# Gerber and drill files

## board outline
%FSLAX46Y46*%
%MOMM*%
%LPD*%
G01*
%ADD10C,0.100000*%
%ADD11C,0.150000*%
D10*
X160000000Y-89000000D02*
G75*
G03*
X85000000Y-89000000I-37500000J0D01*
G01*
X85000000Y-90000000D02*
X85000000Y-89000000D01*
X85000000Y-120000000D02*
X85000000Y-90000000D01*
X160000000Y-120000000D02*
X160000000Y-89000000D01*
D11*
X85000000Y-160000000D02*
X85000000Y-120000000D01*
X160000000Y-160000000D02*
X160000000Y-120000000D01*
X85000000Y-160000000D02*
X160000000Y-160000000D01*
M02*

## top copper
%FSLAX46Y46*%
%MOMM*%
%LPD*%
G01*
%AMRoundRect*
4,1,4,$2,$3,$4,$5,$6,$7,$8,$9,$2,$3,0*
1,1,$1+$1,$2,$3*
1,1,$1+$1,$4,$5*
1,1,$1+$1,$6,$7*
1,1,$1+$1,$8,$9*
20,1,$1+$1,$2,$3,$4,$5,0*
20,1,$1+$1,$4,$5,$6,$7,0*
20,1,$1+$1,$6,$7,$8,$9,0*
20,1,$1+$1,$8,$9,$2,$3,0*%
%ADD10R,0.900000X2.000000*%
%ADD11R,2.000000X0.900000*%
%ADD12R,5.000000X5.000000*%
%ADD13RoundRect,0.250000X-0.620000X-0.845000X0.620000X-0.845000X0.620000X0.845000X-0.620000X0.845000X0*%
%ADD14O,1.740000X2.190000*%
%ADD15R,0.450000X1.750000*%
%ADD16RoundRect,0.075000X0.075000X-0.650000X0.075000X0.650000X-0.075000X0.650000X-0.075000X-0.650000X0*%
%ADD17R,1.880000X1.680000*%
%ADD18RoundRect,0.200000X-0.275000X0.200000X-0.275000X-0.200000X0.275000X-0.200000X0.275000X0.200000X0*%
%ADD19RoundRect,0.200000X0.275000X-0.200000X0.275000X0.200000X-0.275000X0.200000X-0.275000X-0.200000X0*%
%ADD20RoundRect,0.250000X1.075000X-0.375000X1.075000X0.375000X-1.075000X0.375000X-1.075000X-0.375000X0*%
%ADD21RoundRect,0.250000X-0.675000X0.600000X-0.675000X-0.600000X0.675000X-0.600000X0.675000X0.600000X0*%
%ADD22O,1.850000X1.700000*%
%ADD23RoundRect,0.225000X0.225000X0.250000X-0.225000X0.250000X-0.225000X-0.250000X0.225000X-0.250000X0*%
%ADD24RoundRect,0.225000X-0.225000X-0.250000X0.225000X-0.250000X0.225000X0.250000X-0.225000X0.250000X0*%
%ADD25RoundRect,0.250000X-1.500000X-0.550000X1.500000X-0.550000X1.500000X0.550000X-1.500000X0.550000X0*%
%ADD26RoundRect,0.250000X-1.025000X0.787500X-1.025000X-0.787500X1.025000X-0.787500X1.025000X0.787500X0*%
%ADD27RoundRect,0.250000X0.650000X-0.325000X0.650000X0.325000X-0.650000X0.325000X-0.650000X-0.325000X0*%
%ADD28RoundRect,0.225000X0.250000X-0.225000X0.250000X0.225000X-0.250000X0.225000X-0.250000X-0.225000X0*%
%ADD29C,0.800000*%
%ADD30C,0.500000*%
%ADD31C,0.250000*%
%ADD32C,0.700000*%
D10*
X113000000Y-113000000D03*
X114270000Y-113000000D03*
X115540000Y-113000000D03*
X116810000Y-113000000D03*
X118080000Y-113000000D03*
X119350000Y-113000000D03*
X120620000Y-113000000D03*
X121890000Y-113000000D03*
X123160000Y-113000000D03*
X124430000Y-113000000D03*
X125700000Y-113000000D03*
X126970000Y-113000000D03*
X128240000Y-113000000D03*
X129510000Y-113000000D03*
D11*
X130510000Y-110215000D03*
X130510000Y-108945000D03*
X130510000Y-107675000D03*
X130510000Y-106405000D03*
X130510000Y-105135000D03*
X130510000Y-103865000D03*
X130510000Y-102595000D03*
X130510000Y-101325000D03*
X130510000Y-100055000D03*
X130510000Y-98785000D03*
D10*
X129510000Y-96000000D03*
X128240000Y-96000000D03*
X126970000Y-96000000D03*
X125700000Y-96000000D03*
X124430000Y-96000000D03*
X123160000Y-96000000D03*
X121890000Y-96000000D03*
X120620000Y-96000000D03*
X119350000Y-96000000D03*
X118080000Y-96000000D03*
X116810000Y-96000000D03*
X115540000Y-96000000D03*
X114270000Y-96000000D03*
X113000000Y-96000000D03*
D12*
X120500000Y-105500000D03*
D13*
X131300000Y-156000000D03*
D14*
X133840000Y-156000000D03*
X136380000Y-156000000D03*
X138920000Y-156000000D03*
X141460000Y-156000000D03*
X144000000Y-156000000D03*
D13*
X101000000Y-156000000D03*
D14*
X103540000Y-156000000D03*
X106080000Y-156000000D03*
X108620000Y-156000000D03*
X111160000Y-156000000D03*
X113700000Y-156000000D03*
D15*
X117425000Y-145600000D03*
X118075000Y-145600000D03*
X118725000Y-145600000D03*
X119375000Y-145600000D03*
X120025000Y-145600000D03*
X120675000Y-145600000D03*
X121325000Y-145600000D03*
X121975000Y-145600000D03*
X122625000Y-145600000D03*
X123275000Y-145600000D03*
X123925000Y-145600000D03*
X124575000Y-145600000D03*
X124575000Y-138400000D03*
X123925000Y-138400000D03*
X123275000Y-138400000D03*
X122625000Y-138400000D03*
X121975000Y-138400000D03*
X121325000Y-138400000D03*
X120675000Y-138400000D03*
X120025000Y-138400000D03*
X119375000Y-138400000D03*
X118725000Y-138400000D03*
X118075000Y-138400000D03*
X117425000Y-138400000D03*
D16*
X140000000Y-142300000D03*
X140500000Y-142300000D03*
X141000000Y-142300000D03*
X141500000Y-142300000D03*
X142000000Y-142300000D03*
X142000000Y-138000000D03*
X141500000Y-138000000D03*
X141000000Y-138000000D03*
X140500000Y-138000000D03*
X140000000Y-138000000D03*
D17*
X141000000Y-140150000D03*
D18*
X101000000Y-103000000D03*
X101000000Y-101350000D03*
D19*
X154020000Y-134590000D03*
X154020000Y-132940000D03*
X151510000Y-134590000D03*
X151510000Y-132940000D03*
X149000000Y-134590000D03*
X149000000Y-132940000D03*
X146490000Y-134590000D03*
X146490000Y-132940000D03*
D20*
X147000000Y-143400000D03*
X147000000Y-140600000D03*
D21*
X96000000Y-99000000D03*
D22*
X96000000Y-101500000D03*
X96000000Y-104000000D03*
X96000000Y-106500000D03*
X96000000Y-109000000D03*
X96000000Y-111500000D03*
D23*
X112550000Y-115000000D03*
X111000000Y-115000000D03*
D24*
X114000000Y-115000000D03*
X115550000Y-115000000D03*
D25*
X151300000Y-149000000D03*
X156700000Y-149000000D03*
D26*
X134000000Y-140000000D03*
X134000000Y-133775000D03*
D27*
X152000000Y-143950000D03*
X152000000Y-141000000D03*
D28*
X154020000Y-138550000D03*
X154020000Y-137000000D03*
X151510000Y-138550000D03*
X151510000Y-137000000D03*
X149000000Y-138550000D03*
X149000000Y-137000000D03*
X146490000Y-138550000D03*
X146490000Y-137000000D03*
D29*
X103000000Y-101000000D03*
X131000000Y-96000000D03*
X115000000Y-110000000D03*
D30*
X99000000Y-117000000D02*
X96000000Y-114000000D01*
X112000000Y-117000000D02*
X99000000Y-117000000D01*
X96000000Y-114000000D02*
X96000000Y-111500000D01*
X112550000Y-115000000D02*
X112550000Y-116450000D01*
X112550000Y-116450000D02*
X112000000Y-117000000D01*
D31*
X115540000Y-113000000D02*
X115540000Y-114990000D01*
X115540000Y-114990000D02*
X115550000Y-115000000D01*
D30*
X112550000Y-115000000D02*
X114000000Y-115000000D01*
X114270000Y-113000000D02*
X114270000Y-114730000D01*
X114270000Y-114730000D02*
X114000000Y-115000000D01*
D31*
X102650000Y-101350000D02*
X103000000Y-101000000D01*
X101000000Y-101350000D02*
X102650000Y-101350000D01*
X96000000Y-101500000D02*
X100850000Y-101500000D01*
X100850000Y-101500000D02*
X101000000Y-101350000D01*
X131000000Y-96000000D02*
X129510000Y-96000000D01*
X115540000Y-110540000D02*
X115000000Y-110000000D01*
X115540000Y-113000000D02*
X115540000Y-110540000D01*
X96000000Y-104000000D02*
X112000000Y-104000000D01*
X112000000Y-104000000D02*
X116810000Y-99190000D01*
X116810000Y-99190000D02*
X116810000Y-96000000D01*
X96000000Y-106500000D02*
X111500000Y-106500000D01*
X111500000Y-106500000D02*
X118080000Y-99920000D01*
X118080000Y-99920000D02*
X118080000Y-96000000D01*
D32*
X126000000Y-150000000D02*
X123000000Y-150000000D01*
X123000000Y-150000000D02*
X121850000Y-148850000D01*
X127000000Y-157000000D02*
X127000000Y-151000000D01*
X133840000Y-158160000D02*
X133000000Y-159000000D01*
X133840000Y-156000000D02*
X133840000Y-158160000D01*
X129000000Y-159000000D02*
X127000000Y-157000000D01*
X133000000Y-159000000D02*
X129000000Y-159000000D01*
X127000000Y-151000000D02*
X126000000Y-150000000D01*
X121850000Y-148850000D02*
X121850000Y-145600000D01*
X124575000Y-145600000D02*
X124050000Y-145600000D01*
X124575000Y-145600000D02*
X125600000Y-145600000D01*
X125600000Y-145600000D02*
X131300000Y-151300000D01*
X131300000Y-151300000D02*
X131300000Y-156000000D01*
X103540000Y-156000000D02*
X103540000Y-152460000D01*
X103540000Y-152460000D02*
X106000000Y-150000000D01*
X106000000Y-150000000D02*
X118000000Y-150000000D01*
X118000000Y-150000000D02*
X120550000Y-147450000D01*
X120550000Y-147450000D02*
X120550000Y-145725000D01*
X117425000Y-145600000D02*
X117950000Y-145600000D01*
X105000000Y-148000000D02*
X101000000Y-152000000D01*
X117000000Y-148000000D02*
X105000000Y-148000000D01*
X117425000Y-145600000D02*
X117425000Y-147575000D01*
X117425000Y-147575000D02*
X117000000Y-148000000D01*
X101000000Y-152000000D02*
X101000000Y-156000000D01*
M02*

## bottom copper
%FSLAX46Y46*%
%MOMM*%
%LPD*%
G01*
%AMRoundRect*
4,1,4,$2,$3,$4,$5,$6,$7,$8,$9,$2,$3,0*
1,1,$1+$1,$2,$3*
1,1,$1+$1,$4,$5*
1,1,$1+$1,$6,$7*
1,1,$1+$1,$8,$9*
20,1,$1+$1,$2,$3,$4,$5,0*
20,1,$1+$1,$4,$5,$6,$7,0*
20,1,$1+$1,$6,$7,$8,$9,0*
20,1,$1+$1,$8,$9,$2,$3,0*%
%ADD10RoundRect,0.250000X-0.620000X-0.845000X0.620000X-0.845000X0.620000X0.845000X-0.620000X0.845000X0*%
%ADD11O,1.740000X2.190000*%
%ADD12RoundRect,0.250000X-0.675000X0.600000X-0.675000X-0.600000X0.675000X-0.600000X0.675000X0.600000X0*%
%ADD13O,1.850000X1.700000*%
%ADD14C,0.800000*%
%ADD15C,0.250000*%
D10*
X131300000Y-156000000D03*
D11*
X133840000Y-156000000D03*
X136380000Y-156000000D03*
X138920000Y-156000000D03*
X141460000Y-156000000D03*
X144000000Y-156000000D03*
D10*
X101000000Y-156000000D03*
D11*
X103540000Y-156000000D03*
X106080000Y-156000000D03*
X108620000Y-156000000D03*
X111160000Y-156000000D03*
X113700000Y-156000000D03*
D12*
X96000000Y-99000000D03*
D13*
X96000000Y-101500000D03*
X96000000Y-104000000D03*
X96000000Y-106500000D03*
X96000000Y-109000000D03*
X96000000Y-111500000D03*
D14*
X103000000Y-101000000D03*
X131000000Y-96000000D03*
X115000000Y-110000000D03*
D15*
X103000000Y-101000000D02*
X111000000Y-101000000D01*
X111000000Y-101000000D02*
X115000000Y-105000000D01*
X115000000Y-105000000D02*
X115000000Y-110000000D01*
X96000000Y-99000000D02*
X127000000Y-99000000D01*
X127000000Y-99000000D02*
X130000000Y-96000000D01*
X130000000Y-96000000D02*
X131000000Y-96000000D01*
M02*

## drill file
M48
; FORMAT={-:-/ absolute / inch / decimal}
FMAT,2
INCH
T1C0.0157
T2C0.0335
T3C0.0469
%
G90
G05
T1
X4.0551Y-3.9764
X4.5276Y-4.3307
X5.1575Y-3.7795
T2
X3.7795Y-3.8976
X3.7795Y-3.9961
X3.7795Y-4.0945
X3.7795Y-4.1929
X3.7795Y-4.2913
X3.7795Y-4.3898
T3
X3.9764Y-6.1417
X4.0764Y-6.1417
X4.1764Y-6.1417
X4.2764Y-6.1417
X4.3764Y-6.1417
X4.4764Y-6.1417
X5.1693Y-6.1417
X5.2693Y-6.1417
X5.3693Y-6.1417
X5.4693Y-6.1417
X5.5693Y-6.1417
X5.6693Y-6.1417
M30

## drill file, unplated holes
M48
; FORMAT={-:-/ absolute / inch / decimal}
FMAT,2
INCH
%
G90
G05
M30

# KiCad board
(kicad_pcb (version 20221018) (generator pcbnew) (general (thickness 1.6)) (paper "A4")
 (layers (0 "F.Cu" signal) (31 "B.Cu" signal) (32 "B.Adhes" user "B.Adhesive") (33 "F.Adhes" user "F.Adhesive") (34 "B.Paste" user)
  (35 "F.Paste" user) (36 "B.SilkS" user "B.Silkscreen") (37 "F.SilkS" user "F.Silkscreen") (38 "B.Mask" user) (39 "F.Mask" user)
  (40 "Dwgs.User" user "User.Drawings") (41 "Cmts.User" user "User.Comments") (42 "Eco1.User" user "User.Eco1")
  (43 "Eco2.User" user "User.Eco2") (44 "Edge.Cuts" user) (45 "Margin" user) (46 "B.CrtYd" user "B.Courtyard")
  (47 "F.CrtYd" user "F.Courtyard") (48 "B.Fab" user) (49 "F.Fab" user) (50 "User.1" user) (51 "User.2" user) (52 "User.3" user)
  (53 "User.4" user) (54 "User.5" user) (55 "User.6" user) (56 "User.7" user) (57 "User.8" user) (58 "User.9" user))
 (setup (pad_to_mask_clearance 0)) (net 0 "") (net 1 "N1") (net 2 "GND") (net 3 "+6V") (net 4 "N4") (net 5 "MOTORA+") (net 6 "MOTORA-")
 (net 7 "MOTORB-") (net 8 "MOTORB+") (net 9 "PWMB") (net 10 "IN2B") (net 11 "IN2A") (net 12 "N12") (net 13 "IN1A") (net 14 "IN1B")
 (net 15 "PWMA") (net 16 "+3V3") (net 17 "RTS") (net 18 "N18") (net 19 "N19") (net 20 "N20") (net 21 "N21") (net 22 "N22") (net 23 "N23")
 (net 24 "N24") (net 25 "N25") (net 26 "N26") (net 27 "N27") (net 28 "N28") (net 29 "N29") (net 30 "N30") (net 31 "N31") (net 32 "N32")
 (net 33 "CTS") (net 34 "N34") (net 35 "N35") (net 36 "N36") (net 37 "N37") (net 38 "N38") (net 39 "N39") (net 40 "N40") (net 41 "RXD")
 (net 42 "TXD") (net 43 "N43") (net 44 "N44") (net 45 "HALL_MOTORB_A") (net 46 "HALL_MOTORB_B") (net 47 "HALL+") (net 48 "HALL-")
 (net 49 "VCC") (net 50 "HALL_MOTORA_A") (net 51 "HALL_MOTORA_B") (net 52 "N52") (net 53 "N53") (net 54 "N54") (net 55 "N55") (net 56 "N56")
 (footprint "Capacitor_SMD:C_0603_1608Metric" (layer "F.Cu") (at 146.49 137.775 90)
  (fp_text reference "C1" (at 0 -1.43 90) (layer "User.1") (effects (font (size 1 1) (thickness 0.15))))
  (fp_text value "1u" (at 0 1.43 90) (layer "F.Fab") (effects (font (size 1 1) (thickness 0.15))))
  (pad "1" smd roundrect (at -0.775 0 90) (size 0.9 0.95) (layers "F.Cu" "F.Paste" "F.Mask") (roundrect_rratio 0.25) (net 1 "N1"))
  (pad "2" smd roundrect (at 0.775 0 90) (size 0.9 0.95) (layers "F.Cu" "F.Paste" "F.Mask") (roundrect_rratio 0.25) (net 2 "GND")))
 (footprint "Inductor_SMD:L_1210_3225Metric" (layer "F.Cu") (at 147 142 90)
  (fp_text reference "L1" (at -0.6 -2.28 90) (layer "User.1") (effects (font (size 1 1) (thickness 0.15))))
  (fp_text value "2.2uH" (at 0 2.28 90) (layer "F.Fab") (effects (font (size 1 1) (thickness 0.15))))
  (pad "1" smd roundrect (at -1.4 0 90) (size 1.25 2.65) (layers "F.Cu" "F.Paste" "F.Mask") (roundrect_rratio 0.2) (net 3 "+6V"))
  (pad "2" smd roundrect (at 1.4 0 90) (size 1.25 2.65) (layers "F.Cu" "F.Paste" "F.Mask") (roundrect_rratio 0.2) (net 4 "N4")))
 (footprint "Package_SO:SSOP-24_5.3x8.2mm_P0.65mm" (layer "F.Cu") (at 121 142 90)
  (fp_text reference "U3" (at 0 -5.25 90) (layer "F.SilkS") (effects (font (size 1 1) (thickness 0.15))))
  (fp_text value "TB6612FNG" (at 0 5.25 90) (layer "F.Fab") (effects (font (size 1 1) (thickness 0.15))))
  (pad "1" smd rect (at -3.6 -3.575 90) (size 1.75 0.45) (layers "F.Cu" "F.Paste" "F.Mask") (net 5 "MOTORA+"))
  (pad "2" smd rect (at -3.6 -2.925 90) (size 1.75 0.45) (layers "F.Cu" "F.Paste" "F.Mask") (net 5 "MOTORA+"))
  (pad "3" smd rect (at -3.6 -2.275 90) (size 1.75 0.45) (layers "F.Cu" "F.Paste" "F.Mask") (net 2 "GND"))
  (pad "4" smd rect (at -3.6 -1.625 90) (size 1.75 0.45) (layers "F.Cu" "F.Paste" "F.Mask") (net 2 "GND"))
  (pad "5" smd rect (at -3.6 -0.975 90) (size 1.75 0.45) (layers "F.Cu" "F.Paste" "F.Mask") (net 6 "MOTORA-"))
  (pad "6" smd rect (at -3.6 -0.325 90) (size 1.75 0.45) (layers "F.Cu" "F.Paste" "F.Mask") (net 6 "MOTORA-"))
  (pad "7" smd rect (at -3.6 0.325 90) (size 1.75 0.45) (layers "F.Cu" "F.Paste" "F.Mask") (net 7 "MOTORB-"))
  (pad "8" smd rect (at -3.6 0.975 90) (size 1.75 0.45) (layers "F.Cu" "F.Paste" "F.Mask") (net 7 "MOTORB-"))
  (pad "9" smd rect (at -3.6 1.625 90) (size 1.75 0.45) (layers "F.Cu" "F.Paste" "F.Mask") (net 2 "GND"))
  (pad "10" smd rect (at -3.6 2.275 90) (size 1.75 0.45) (layers "F.Cu" "F.Paste" "F.Mask") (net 2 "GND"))
  (pad "11" smd rect (at -3.6 2.925 90) (size 1.75 0.45) (layers "F.Cu" "F.Paste" "F.Mask") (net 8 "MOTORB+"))
  (pad "12" smd rect (at -3.6 3.575 90) (size 1.75 0.45) (layers "F.Cu" "F.Paste" "F.Mask") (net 8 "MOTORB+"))
  (pad "13" smd rect (at 3.6 3.575 90) (size 1.75 0.45) (layers "F.Cu" "F.Paste" "F.Mask") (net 3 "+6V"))
  (pad "14" smd rect (at 3.6 2.925 90) (size 1.75 0.45) (layers "F.Cu" "F.Paste" "F.Mask") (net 3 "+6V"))
  (pad "15" smd rect (at 3.6 2.275 90) (size 1.75 0.45) (layers "F.Cu" "F.Paste" "F.Mask") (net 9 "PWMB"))
  (pad "16" smd rect (at 3.6 1.625 90) (size 1.75 0.45) (layers "F.Cu" "F.Paste" "F.Mask") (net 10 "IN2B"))
  (pad "17" smd rect (at 3.6 0.975 90) (size 1.75 0.45) (layers "F.Cu" "F.Paste" "F.Mask") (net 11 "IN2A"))
  (pad "18" smd rect (at 3.6 0.325 90) (size 1.75 0.45) (layers "F.Cu" "F.Paste" "F.Mask") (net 2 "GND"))
  (pad "19" smd rect (at 3.6 -0.325 90) (size 1.75 0.45) (layers "F.Cu" "F.Paste" "F.Mask") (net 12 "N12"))
  (pad "20" smd rect (at 3.6 -0.975 90) (size 1.75 0.45) (layers "F.Cu" "F.Paste" "F.Mask") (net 3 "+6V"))
  (pad "21" smd rect (at 3.6 -1.625 90) (size 1.75 0.45) (layers "F.Cu" "F.Paste" "F.Mask") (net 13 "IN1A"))
  (pad "22" smd rect (at 3.6 -2.275 90) (size 1.75 0.45) (layers "F.Cu" "F.Paste" "F.Mask") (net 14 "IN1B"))
  (pad "23" smd rect (at 3.6 -2.925 90) (size 1.75 0.45) (layers "F.Cu" "F.Paste" "F.Mask") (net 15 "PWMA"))
  (pad "24" smd rect (at 3.6 -3.575 90) (size 1.75 0.45) (layers "F.Cu" "F.Paste" "F.Mask") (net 3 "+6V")))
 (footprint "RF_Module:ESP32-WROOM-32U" (layer "F.Cu") (at 121.255 104.5 90)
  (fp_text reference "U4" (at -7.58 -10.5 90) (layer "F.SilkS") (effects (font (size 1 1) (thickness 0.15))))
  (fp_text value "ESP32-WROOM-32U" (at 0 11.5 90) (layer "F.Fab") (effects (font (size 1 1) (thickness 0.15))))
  (pad "1" smd rect (at -8.5 -8.255 90) (size 2 0.9) (layers "F.Cu" "F.Paste" "F.Mask") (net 2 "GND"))
  (pad "2" smd rect (at -8.5 -6.985 90) (size 2 0.9) (layers "F.Cu" "F.Paste" "F.Mask") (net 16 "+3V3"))
  (pad "3" smd rect (at -8.5 -5.715 90) (size 2 0.9) (layers "F.Cu" "F.Paste" "F.Mask") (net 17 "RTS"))
  (pad "4" smd rect (at -8.5 -4.445 90) (size 2 0.9) (layers "F.Cu" "F.Paste" "F.Mask") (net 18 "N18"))
  (pad "5" smd rect (at -8.5 -3.175 90) (size 2 0.9) (layers "F.Cu" "F.Paste" "F.Mask") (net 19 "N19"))
  (pad "6" smd rect (at -8.5 -1.905 90) (size 2 0.9) (layers "F.Cu" "F.Paste" "F.Mask") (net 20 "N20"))
  (pad "7" smd rect (at -8.5 -0.635 90) (size 2 0.9) (layers "F.Cu" "F.Paste" "F.Mask") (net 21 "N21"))
  (pad "8" smd rect (at -8.5 0.635 90) (size 2 0.9) (layers "F.Cu" "F.Paste" "F.Mask") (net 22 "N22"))
  (pad "9" smd rect (at -8.5 1.905 90) (size 2 0.9) (layers "F.Cu" "F.Paste" "F.Mask") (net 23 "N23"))
  (pad "10" smd rect (at -8.5 3.175 90) (size 2 0.9) (layers "F.Cu" "F.Paste" "F.Mask") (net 15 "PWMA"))
  (pad "11" smd rect (at -8.5 4.445 90) (size 2 0.9) (layers "F.Cu" "F.Paste" "F.Mask") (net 14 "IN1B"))
  (pad "12" smd rect (at -8.5 5.715 90) (size 2 0.9) (layers "F.Cu" "F.Paste" "F.Mask") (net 13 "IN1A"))
  (pad "13" smd rect (at -8.5 6.985 90) (size 2 0.9) (layers "F.Cu" "F.Paste" "F.Mask") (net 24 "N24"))
  (pad "14" smd rect (at -8.5 8.255 90) (size 2 0.9) (layers "F.Cu" "F.Paste" "F.Mask") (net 11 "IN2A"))
  (pad "15" smd rect (at -5.715 9.255) (size 2 0.9) (layers "F.Cu" "F.Paste" "F.Mask") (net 2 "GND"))
  (pad "16" smd rect (at -4.445 9.255 180) (size 2 0.9) (layers "F.Cu" "F.Paste" "F.Mask") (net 9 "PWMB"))
  (pad "17" smd rect (at -3.175 9.255 180) (size 2 0.9) (layers "F.Cu" "F.Paste" "F.Mask") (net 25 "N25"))
  (pad "18" smd rect (at -1.905 9.255 180) (size 2 0.9) (layers "F.Cu" "F.Paste" "F.Mask") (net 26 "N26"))
  (pad "19" smd rect (at -0.635 9.255 180) (size 2 0.9) (layers "F.Cu" "F.Paste" "F.Mask") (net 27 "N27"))
  (pad "20" smd rect (at 0.635 9.255 180) (size 2 0.9) (layers "F.Cu" "F.Paste" "F.Mask") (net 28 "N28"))
  (pad "21" smd rect (at 1.905 9.255 180) (size 2 0.9) (layers "F.Cu" "F.Paste" "F.Mask") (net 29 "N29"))
  (pad "22" smd rect (at 3.175 9.255 180) (size 2 0.9) (layers "F.Cu" "F.Paste" "F.Mask") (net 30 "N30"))
  (pad "23" smd rect (at 4.445 9.255 180) (size 2 0.9) (layers "F.Cu" "F.Paste" "F.Mask") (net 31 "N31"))
  (pad "24" smd rect (at 5.715 9.255 180) (size 2 0.9) (layers "F.Cu" "F.Paste" "F.Mask") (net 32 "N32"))
  (pad "25" smd rect (at 8.5 8.255 90) (size 2 0.9) (layers "F.Cu" "F.Paste" "F.Mask") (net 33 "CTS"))
  (pad "26" smd rect (at 8.5 6.985 90) (size 2 0.9) (layers "F.Cu" "F.Paste" "F.Mask") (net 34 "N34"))
  (pad "27" smd rect (at 8.5 5.715 90) (size 2 0.9) (layers "F.Cu" "F.Paste" "F.Mask") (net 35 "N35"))
  (pad "28" smd rect (at 8.5 4.445 90) (size 2 0.9) (layers "F.Cu" "F.Paste" "F.Mask") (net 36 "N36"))
  (pad "29" smd rect (at 8.5 3.175 90) (size 2 0.9) (layers "F.Cu" "F.Paste" "F.Mask") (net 10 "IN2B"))
  (pad "30" smd rect (at 8.5 1.905 90) (size 2 0.9) (layers "F.Cu" "F.Paste" "F.Mask") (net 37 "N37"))
  (pad "31" smd rect (at 8.5 0.635 90) (size 2 0.9) (layers "F.Cu" "F.Paste" "F.Mask") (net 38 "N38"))
  (pad "32" smd rect (at 8.5 -0.635 90) (size 2 0.9) (layers "F.Cu" "F.Paste" "F.Mask") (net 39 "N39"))
  (pad "33" smd rect (at 8.5 -1.905 90) (size 2 0.9) (layers "F.Cu" "F.Paste" "F.Mask") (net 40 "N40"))
  (pad "34" smd rect (at 8.5 -3.175 90) (size 2 0.9) (layers "F.Cu" "F.Paste" "F.Mask") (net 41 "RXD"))
  (pad "35" smd rect (at 8.5 -4.445 90) (size 2 0.9) (layers "F.Cu" "F.Paste" "F.Mask") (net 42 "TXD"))
  (pad "36" smd rect (at 8.5 -5.715 90) (size 2 0.9) (layers "F.Cu" "F.Paste" "F.Mask") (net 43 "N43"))
  (pad "37" smd rect (at 8.5 -6.985 90) (size 2 0.9) (layers "F.Cu" "F.Paste" "F.Mask") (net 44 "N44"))
  (pad "38" smd rect (at 8.5 -8.255 90) (size 2 0.9) (layers "F.Cu" "F.Paste" "F.Mask") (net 2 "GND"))
  (pad "39" smd rect (at -1 -0.755 90) (size 5 5) (layers "F.Cu" "F.Paste" "F.Mask") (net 2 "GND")))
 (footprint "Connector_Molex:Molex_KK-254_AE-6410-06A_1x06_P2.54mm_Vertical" (layer "F.Cu") (at 131.3 156)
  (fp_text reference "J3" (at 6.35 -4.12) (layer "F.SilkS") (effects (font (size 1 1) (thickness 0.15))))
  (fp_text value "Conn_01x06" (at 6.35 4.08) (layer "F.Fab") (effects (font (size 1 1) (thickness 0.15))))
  (pad "1" thru_hole roundrect (at 0 0) (size 1.74 2.19) (drill 1.19) (layers "*.Cu" "*.Mask") (roundrect_rratio 0.1436781609)
   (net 8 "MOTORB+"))
  (pad "2" thru_hole oval (at 2.54 0) (size 1.74 2.19) (drill 1.19) (layers "*.Cu" "*.Mask") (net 7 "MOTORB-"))
  (pad "3" thru_hole oval (at 5.08 0) (size 1.74 2.19) (drill 1.19) (layers "*.Cu" "*.Mask") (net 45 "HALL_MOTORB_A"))
  (pad "4" thru_hole oval (at 7.62 0) (size 1.74 2.19) (drill 1.19) (layers "*.Cu" "*.Mask") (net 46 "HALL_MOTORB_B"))
  (pad "5" thru_hole oval (at 10.16 0) (size 1.74 2.19) (drill 1.19) (layers "*.Cu" "*.Mask") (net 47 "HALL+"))
  (pad "6" thru_hole oval (at 12.7 0) (size 1.74 2.19) (drill 1.19) (layers "*.Cu" "*.Mask") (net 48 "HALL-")))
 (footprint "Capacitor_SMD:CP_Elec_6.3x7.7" (layer "F.Cu") (at 154 149)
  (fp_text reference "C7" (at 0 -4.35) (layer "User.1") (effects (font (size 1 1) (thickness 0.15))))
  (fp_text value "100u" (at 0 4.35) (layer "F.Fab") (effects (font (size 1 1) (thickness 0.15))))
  (pad "1" smd roundrect (at -2.7 0) (size 3.5 1.6) (layers "F.Cu" "F.Paste" "F.Mask") (roundrect_rratio 0.15625) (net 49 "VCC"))
  (pad "2" smd roundrect (at 2.7 0) (size 3.5 1.6) (layers "F.Cu" "F.Paste" "F.Mask") (roundrect_rratio 0.15625) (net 2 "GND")))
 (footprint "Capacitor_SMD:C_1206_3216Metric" (layer "F.Cu") (at 152 142.475 90)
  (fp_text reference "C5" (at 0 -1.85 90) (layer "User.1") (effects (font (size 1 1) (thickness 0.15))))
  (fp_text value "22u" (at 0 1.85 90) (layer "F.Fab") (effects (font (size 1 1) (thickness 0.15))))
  (pad "1" smd roundrect (at -1.475 0 90) (size 1.15 1.8) (layers "F.Cu" "F.Paste" "F.Mask") (roundrect_rratio 0.2173913043) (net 3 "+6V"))
  (pad "2" smd roundrect (at 1.475 0 90) (size 1.15 1.8) (layers "F.Cu" "F.Paste" "F.Mask") (roundrect_rratio 0.2173913043) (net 2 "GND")))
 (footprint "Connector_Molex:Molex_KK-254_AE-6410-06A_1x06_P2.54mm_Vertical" (layer "F.Cu") (at 101 156)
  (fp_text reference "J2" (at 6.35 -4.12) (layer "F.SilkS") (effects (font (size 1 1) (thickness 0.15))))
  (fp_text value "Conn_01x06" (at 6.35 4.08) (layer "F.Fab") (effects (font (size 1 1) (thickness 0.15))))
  (pad "1" thru_hole roundrect (at 0 0) (size 1.74 2.19) (drill 1.19) (layers "*.Cu" "*.Mask") (roundrect_rratio 0.1436781609)
   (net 5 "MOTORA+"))
  (pad "2" thru_hole oval (at 2.54 0) (size 1.74 2.19) (drill 1.19) (layers "*.Cu" "*.Mask") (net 6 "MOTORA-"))
  (pad "3" thru_hole oval (at 5.08 0) (size 1.74 2.19) (drill 1.19) (layers "*.Cu" "*.Mask") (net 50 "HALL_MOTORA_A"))
  (pad "4" thru_hole oval (at 7.62 0) (size 1.74 2.19) (drill 1.19) (layers "*.Cu" "*.Mask") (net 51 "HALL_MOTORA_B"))
  (pad "5" thru_hole oval (at 10.16 0) (size 1.74 2.19) (drill 1.19) (layers "*.Cu" "*.Mask") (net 47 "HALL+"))
  (pad "6" thru_hole oval (at 12.7 0) (size 1.74 2.19) (drill 1.19) (layers "*.Cu" "*.Mask") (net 48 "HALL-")))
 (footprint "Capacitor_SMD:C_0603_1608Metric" (layer "F.Cu") (at 149 137.775 90)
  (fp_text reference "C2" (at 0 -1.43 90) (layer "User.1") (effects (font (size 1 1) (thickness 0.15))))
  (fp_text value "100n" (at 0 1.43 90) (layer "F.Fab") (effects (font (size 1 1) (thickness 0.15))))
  (pad "1" smd roundrect (at -0.775 0 90) (size 0.9 0.95) (layers "F.Cu" "F.Paste" "F.Mask") (roundrect_rratio 0.25) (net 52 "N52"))
  (pad "2" smd roundrect (at 0.775 0 90) (size 0.9 0.95) (layers "F.Cu" "F.Paste" "F.Mask") (roundrect_rratio 0.25) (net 4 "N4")))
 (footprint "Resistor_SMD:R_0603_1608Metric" (layer "F.Cu") (at 149 133.765 90)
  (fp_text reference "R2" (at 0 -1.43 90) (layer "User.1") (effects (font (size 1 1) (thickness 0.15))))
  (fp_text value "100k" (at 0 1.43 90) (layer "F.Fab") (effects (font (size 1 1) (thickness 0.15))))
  (pad "1" smd roundrect (at -0.825 0 90) (size 0.8 0.95) (layers "F.Cu" "F.Paste" "F.Mask") (roundrect_rratio 0.25) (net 3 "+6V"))
  (pad "2" smd roundrect (at 0.825 0 90) (size 0.8 0.95) (layers "F.Cu" "F.Paste" "F.Mask") (roundrect_rratio 0.25) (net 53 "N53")))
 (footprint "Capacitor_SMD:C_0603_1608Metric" (layer "F.Cu") (at 154.02 137.775 90)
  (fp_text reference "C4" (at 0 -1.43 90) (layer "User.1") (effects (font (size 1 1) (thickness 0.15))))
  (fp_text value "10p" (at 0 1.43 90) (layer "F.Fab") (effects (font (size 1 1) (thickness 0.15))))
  (pad "1" smd roundrect (at -0.775 0 90) (size 0.9 0.95) (layers "F.Cu" "F.Paste" "F.Mask") (roundrect_rratio 0.25) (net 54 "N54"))
  (pad "2" smd roundrect (at 0.775 0 90) (size 0.9 0.95) (layers "F.Cu" "F.Paste" "F.Mask") (roundrect_rratio 0.25) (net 3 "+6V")))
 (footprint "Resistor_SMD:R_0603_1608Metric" (layer "F.Cu") (at 101 102.175 -90)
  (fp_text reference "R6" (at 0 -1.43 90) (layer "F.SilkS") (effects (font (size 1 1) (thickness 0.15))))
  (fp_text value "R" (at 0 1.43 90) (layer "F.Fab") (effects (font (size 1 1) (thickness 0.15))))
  (pad "1" smd roundrect (at -0.825 0 270) (size 0.8 0.95) (layers "F.Cu" "F.Paste" "F.Mask") (roundrect_rratio 0.25) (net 17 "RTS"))
  (pad "2" smd roundrect (at 0.825 0 270) (size 0.8 0.95) (layers "F.Cu" "F.Paste" "F.Mask") (roundrect_rratio 0.25) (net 2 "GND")))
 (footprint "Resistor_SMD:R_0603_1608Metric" (layer "F.Cu") (at 154.02 133.765 90)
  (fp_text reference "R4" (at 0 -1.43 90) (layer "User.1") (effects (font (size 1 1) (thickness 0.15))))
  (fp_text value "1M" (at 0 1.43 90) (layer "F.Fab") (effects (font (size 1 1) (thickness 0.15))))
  (pad "1" smd roundrect (at -0.825 0 90) (size 0.8 0.95) (layers "F.Cu" "F.Paste" "F.Mask") (roundrect_rratio 0.25) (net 3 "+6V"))
  (pad "2" smd roundrect (at 0.825 0 90) (size 0.8 0.95) (layers "F.Cu" "F.Paste" "F.Mask") (roundrect_rratio 0.25) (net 54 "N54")))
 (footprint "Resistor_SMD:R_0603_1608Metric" (layer "F.Cu") (at 146.49 133.765 90)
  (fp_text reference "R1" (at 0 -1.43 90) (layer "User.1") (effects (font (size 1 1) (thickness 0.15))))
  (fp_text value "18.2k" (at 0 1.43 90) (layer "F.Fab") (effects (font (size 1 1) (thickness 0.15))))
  (pad "1" smd roundrect (at -0.825 0 90) (size 0.8 0.95) (layers "F.Cu" "F.Paste" "F.Mask") (roundrect_rratio 0.25) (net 2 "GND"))
  (pad "2" smd roundrect (at 0.825 0 90) (size 0.8 0.95) (layers "F.Cu" "F.Paste" "F.Mask") (roundrect_rratio 0.25) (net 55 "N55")))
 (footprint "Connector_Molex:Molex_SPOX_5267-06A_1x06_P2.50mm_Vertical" (layer "F.Cu") (at 96 99 -90)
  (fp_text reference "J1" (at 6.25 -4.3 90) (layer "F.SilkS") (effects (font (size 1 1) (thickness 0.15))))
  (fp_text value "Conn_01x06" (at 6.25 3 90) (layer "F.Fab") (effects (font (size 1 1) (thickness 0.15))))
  (pad "1" thru_hole roundrect (at 0 0 270) (size 1.7 1.85) (drill 0.85) (layers "*.Cu" "*.Mask") (roundrect_rratio 0.1470588235)
   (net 33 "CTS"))
  (pad "2" thru_hole oval (at 2.5 0 270) (size 1.7 1.85) (drill 0.85) (layers "*.Cu" "*.Mask") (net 17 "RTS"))
  (pad "3" thru_hole oval (at 5 0 270) (size 1.7 1.85) (drill 0.85) (layers "*.Cu" "*.Mask") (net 42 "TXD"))
  (pad "4" thru_hole oval (at 7.5 0 270) (size 1.7 1.85) (drill 0.85) (layers "*.Cu" "*.Mask") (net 41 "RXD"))
  (pad "5" thru_hole oval (at 10 0 270) (size 1.7 1.85) (drill 0.85) (layers "*.Cu" "*.Mask") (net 2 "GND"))
  (pad "6" thru_hole oval (at 12.5 0 270) (size 1.7 1.85) (drill 0.85) (layers "*.Cu" "*.Mask") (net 16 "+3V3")))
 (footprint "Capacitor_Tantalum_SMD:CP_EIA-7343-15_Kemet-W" (layer "F.Cu") (at 134 136.8875 -90)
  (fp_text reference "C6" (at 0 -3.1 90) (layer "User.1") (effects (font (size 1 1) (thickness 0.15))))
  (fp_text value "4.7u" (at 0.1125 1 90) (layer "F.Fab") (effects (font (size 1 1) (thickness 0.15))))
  (pad "1" smd roundrect (at -3.1125 0 270) (size 2.075 2.55) (layers "F.Cu" "F.Paste" "F.Mask") (roundrect_rratio 0.1204819277)
   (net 49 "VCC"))
  (pad "2" smd roundrect (at 3.1125 0 270) (size 2.075 2.55) (layers "F.Cu" "F.Paste" "F.Mask") (roundrect_rratio 0.1204819277)
   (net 2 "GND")))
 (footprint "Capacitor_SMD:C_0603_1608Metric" (layer "F.Cu") (at 114.775 115)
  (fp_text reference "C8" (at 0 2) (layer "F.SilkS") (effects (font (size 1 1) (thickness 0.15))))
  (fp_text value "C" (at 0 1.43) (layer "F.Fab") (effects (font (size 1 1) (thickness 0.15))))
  (pad "1" smd roundrect (at -0.775 0) (size 0.9 0.95) (layers "F.Cu" "F.Paste" "F.Mask") (roundrect_rratio 0.25) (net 16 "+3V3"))
  (pad "2" smd roundrect (at 0.775 0) (size 0.9 0.95) (layers "F.Cu" "F.Paste" "F.Mask") (roundrect_rratio 0.25) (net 17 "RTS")))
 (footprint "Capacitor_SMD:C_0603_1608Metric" (layer "F.Cu") (at 111.775 115 180)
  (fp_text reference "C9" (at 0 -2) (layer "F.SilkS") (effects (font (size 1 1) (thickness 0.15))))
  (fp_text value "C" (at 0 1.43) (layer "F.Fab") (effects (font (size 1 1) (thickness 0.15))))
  (pad "1" smd roundrect (at -0.775 0 180) (size 0.9 0.95) (layers "F.Cu" "F.Paste" "F.Mask") (roundrect_rratio 0.25) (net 16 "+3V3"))
  (pad "2" smd roundrect (at 0.775 0 180) (size 0.9 0.95) (layers "F.Cu" "F.Paste" "F.Mask") (roundrect_rratio 0.25) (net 2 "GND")))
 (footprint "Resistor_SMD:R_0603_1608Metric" (layer "F.Cu") (at 151.51 133.765 90)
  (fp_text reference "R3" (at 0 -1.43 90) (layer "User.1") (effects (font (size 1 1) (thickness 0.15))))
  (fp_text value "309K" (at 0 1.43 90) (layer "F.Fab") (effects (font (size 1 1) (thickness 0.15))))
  (pad "1" smd roundrect (at -0.825 0 90) (size 0.8 0.95) (layers "F.Cu" "F.Paste" "F.Mask") (roundrect_rratio 0.25) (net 2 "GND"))
  (pad "2" smd roundrect (at 0.825 0 90) (size 0.8 0.95) (layers "F.Cu" "F.Paste" "F.Mask") (roundrect_rratio 0.25) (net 54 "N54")))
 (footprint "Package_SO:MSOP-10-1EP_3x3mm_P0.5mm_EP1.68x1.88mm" (layer "F.Cu") (at 141 140.15 90)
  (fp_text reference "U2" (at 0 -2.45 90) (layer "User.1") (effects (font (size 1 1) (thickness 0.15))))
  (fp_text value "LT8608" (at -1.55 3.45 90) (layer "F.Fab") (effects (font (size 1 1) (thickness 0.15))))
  (pad "" smd roundrect (at -0.42 -0.47 90) (size 0.68 0.76) (layers "F.Paste") (roundrect_rratio 0.25))
  (pad "" smd roundrect (at -0.42 0.47 90) (size 0.68 0.76) (layers "F.Paste") (roundrect_rratio 0.25))
  (pad "" smd roundrect (at 0.42 -0.47 90) (size 0.68 0.76) (layers "F.Paste") (roundrect_rratio 0.25))
  (pad "" smd roundrect (at 0.42 0.47 90) (size 0.68 0.76) (layers "F.Paste") (roundrect_rratio 0.25))
  (pad "1" smd roundrect (at -2.15 -1 90) (size 1.45 0.3) (layers "F.Cu" "F.Paste" "F.Mask") (roundrect_rratio 0.25) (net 52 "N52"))
  (pad "2" smd roundrect (at -2.15 -0.5 90) (size 1.45 0.3) (layers "F.Cu" "F.Paste" "F.Mask") (roundrect_rratio 0.25) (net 4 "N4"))
  (pad "3" smd roundrect (at -2.15 0 90) (size 1.45 0.3) (layers "F.Cu" "F.Paste" "F.Mask") (roundrect_rratio 0.25) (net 1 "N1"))
  (pad "4" smd roundrect (at -2.15 0.5 90) (size 1.45 0.3) (layers "F.Cu" "F.Paste" "F.Mask") (roundrect_rratio 0.25) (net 55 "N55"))
  (pad "5" smd roundrect (at -2.15 1 90) (size 1.45 0.3) (layers "F.Cu" "F.Paste" "F.Mask") (roundrect_rratio 0.25) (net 2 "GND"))
  (pad "6" smd roundrect (at 2.15 1 90) (size 1.45 0.3) (layers "F.Cu" "F.Paste" "F.Mask") (roundrect_rratio 0.25) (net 54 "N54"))
  (pad "7" smd roundrect (at 2.15 0.5 90) (size 1.45 0.3) (layers "F.Cu" "F.Paste" "F.Mask") (roundrect_rratio 0.25) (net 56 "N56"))
  (pad "8" smd roundrect (at 2.15 0 90) (size 1.45 0.3) (layers "F.Cu" "F.Paste" "F.Mask") (roundrect_rratio 0.25) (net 53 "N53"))
  (pad "9" smd roundrect (at 2.15 -0.5 90) (size 1.45 0.3) (layers "F.Cu" "F.Paste" "F.Mask") (roundrect_rratio 0.25) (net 49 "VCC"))
  (pad "10" smd roundrect (at 2.15 -1 90) (size 1.45 0.3) (layers "F.Cu" "F.Paste" "F.Mask") (roundrect_rratio 0.25) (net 49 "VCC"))
  (pad "11" smd rect (at 0 0 90) (size 1.68 1.88) (layers "F.Cu" "F.Mask") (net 2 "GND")))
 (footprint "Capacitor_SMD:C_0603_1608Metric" (layer "F.Cu") (at 151.51 137.775 90)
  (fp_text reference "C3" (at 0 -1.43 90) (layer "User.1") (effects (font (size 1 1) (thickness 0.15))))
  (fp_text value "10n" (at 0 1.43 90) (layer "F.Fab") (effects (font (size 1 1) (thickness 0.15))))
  (pad "1" smd roundrect (at -0.775 0 90) (size 0.9 0.95) (layers "F.Cu" "F.Paste" "F.Mask") (roundrect_rratio 0.25) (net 56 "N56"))
  (pad "2" smd roundrect (at 0.775 0 90) (size 0.9 0.95) (layers "F.Cu" "F.Paste" "F.Mask") (roundrect_rratio 0.25) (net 2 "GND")))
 (gr_line (start 85 90) (end 85 89) (stroke (width 0.1) (type default)) (layer "Edge.Cuts"))
 (gr_arc (start 85 89) (mid 122.5 51.5) (end 160 89) (stroke (width 0.1) (type default)) (layer "Edge.Cuts"))
 (gr_line (start 85 160) (end 160 160) (stroke (width 0.15) (type default)) (layer "Edge.Cuts"))
 (gr_line (start 85 160) (end 85 120) (stroke (width 0.15) (type default)) (layer "Edge.Cuts"))
 (gr_line (start 160 120) (end 160 89) (stroke (width 0.1) (type default)) (layer "Edge.Cuts"))
 (gr_line (start 85 120) (end 85 90) (stroke (width 0.1) (type default)) (layer "Edge.Cuts"))
 (gr_line (start 160 160) (end 160 120) (stroke (width 0.15) (type default)) (layer "Edge.Cuts"))
 (segment (start 112.55 115) (end 114 115) (width 0.5) (layer "F.Cu") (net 16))
 (segment (start 112.55 115) (end 112.55 116.45) (width 0.5) (layer "F.Cu") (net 16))
 (segment (start 112 117) (end 99 117) (width 0.5) (layer "F.Cu") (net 16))
 (segment (start 99 117) (end 96 114) (width 0.5) (layer "F.Cu") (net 16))
 (segment (start 96 114) (end 96 111.5) (width 0.5) (layer "F.Cu") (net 16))
 (segment (start 114.27 114.73) (end 114 115) (width 0.5) (layer "F.Cu") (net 16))
 (segment (start 112.55 116.45) (end 112 117) (width 0.5) (layer "F.Cu") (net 16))
 (segment (start 114.27 113) (end 114.27 114.73) (width 0.5) (layer "F.Cu") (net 16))
 (segment (start 102.65 101.35) (end 103 101) (width 0.25) (layer "F.Cu") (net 17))
 (segment (start 115.54 113) (end 115.54 114.99) (width 0.25) (layer "F.Cu") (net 17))
 (segment (start 115.54 113) (end 115.54 110.54) (width 0.25) (layer "F.Cu") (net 17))
 (segment (start 101 101.35) (end 102.65 101.35) (width 0.25) (layer "F.Cu") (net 17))
 (segment (start 100.85 101.5) (end 101 101.35) (width 0.25) (layer "F.Cu") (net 17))
 (segment (start 115.54 114.99) (end 115.55 115) (width 0.25) (layer "F.Cu") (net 17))
 (segment (start 96 101.5) (end 100.85 101.5) (width 0.25) (layer "F.Cu") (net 17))
 (segment (start 115.54 110.54) (end 115 110) (width 0.25) (layer "F.Cu") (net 17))
 (via (at 103 101) (size 0.8) (drill 0.4) (layers "F.Cu" "B.Cu") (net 17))
 (via (at 115 110) (size 0.8) (drill 0.4) (layers "F.Cu" "B.Cu") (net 17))
 (segment (start 111 101) (end 115 105) (width 0.25) (layer "B.Cu") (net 17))
 (segment (start 115 105) (end 115 110) (width 0.25) (layer "B.Cu") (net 17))
 (segment (start 103 101) (end 111 101) (width 0.25) (layer "B.Cu") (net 17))
 (segment (start 131 96) (end 129.51 96) (width 0.25) (layer "F.Cu") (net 33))
 (via (at 131 96) (size 0.8) (drill 0.4) (layers "F.Cu" "B.Cu") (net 33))
 (segment (start 96 99) (end 127 99) (width 0.25) (layer "B.Cu") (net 33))
 (segment (start 130 96) (end 131 96) (width 0.25) (layer "B.Cu") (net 33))
 (segment (start 127 99) (end 130 96) (width 0.25) (layer "B.Cu") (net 33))
 (segment (start 96 104) (end 112 104) (width 0.25) (layer "F.Cu") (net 42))
 (segment (start 116.81 99.19) (end 116.81 96) (width 0.25) (layer "F.Cu") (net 42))
 (segment (start 112 104) (end 116.81 99.19) (width 0.25) (layer "F.Cu") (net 42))
 (segment (start 111.5 106.5) (end 118.08 99.92) (width 0.25) (layer "F.Cu") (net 41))
 (segment (start 96 106.5) (end 111.5 106.5) (width 0.25) (layer "F.Cu") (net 41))
 (segment (start 118.08 99.92) (end 118.08 96) (width 0.25) (layer "F.Cu") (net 41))
 (segment (start 105 148) (end 101 152) (width 0.7) (layer "F.Cu") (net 5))
 (segment (start 117.425 145.6) (end 117.425 147.575) (width 0.7) (layer "F.Cu") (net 5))
 (segment (start 101 152) (end 101 156) (width 0.7) (layer "F.Cu") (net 5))
 (segment (start 117.425 147.575) (end 117 148) (width 0.7) (layer "F.Cu") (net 5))
 (segment (start 117 148) (end 105 148) (width 0.7) (layer "F.Cu") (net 5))
 (segment (start 117.425 145.6) (end 117.95 145.6) (width 0.7) (layer "F.Cu") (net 5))
 (segment (start 120.55 147.45) (end 120.55 145.725) (width 0.7) (layer "F.Cu") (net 6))
 (segment (start 103.54 156) (end 103.54 152.46) (width 0.7) (layer "F.Cu") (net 6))
 (segment (start 118 150) (end 120.55 147.45) (width 0.7) (layer "F.Cu") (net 6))
 (segment (start 103.54 152.46) (end 106 150) (width 0.7) (layer "F.Cu") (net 6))
 (segment (start 106 150) (end 118 150) (width 0.7) (layer "F.Cu") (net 6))
 (segment (start 124.575 145.6) (end 125.6 145.6) (width 0.7) (layer "F.Cu") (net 8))
 (segment (start 124.575 145.6) (end 124.05 145.6) (width 0.7) (layer "F.Cu") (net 8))
 (segment (start 131.3 151.3) (end 131.3 156) (width 0.7) (layer "F.Cu") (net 8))
 (segment (start 125.6 145.6) (end 131.3 151.3) (width 0.7) (layer "F.Cu") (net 8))
 (segment (start 126 150) (end 123 150) (width 0.7) (layer "F.Cu") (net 7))
 (segment (start 127 157) (end 127 151) (width 0.7) (layer "F.Cu") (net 7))
 (segment (start 121.85 148.85) (end 121.85 145.6) (width 0.7) (layer "F.Cu") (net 7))
 (segment (start 123 150) (end 121.85 148.85) (width 0.7) (layer "F.Cu") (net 7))
 (segment (start 129 159) (end 127 157) (width 0.7) (layer "F.Cu") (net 7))
 (segment (start 133.84 158.16) (end 133 159) (width 0.7) (layer "F.Cu") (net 7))
 (segment (start 133.84 156) (end 133.84 158.16) (width 0.7) (layer "F.Cu") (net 7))
 (segment (start 133 159) (end 129 159) (width 0.7) (layer "F.Cu") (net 7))
 (segment (start 127 151) (end 126 150) (width 0.7) (layer "F.Cu") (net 7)))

